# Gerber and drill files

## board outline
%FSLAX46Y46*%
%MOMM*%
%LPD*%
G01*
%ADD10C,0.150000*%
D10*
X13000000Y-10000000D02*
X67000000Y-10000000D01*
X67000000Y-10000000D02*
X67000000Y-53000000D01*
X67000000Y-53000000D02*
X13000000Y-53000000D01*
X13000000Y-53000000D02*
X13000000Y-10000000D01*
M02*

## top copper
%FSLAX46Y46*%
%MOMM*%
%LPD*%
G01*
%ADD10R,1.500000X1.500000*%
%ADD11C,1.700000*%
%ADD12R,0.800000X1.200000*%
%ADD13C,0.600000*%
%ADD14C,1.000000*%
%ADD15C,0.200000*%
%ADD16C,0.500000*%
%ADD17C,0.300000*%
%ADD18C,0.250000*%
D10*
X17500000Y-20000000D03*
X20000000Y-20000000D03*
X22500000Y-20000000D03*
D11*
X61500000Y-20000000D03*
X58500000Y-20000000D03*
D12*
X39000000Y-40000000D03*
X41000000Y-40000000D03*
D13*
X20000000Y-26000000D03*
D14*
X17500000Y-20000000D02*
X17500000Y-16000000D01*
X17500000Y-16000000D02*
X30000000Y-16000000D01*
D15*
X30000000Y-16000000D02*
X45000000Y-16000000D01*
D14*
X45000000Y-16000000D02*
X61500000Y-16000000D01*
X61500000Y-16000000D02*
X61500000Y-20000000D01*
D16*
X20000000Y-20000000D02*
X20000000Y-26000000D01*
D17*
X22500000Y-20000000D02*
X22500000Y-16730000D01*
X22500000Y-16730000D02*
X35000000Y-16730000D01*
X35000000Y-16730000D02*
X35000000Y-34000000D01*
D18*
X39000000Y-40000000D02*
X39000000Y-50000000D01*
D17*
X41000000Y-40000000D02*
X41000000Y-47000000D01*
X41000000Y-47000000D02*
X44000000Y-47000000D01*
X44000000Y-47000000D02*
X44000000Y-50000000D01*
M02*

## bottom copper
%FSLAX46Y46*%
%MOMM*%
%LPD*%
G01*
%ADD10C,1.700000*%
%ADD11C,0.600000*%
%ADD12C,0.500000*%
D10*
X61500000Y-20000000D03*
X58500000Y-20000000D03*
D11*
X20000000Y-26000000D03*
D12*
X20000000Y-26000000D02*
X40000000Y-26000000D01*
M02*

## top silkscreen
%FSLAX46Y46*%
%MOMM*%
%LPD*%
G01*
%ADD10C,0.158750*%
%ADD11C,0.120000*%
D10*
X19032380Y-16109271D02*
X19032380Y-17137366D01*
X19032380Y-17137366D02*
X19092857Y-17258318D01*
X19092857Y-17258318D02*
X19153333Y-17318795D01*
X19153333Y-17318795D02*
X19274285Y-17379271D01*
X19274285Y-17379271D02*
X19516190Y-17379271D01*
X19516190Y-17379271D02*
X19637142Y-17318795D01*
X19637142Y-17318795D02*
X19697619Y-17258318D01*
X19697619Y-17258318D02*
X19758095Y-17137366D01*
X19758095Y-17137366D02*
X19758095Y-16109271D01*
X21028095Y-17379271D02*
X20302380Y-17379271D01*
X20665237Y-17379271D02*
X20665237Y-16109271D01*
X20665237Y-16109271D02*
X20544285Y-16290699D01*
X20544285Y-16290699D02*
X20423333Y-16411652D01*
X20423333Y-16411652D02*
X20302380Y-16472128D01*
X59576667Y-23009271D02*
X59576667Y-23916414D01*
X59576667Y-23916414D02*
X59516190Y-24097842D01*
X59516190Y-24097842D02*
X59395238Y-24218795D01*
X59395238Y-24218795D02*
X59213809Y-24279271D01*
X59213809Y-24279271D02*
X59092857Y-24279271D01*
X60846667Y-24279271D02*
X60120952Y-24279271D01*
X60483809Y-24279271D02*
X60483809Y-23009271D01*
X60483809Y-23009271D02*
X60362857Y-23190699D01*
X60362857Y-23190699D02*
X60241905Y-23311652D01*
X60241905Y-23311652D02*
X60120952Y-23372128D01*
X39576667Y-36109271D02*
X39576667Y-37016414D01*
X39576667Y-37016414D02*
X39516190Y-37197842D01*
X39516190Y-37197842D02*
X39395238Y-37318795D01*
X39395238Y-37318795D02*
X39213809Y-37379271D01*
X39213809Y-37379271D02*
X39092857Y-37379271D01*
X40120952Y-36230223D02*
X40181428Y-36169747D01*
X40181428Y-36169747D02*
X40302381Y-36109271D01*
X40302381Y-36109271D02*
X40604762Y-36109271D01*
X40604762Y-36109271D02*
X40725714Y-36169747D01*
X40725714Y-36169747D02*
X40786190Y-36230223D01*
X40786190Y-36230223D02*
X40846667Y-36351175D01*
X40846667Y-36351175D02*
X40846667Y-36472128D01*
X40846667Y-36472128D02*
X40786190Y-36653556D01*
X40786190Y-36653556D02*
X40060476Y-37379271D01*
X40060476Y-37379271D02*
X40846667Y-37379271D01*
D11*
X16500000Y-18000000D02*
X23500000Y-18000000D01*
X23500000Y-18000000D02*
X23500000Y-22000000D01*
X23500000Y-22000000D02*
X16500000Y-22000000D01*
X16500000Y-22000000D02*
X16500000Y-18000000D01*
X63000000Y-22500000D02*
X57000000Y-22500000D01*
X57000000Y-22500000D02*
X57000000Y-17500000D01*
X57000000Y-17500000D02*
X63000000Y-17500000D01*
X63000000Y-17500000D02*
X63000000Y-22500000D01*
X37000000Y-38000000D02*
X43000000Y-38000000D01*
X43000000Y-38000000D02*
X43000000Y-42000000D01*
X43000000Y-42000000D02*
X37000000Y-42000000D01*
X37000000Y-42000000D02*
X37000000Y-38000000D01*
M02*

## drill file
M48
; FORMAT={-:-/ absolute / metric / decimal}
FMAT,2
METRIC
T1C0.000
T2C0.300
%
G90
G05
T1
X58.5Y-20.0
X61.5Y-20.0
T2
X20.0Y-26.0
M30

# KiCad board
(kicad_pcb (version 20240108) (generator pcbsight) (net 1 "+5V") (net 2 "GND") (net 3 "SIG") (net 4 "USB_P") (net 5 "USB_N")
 (gr_line (start 13 10) (end 67 10) (layer "Edge.Cuts") (width 0.15))
 (gr_line (start 67 10) (end 67 53) (layer "Edge.Cuts") (width 0.15))
 (gr_line (start 67 53) (end 13 53) (layer "Edge.Cuts") (width 0.15))
 (gr_line (start 13 53) (end 13 10) (layer "Edge.Cuts") (width 0.15))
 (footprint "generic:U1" (at 20 20 0) (layer "F.Cu") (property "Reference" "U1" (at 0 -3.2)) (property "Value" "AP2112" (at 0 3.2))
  (fp_line (start -3.5 -2.0) (end 3.5 -2.0) (layer "F.SilkS") (width 0.12))
  (fp_line (start 3.5 -2.0) (end 3.5 2.0) (layer "F.SilkS") (width 0.12))
  (fp_line (start 3.5 2.0) (end -3.5 2.0) (layer "F.SilkS") (width 0.12))
  (fp_line (start -3.5 2.0) (end -3.5 -2.0) (layer "F.SilkS") (width 0.12))
  (pad "1" smd rect (at -2.5 0) (size 1.5 1.5) (layers "F.Cu" "F.Mask") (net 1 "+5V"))
  (pad "2" smd rect (at 0 0) (size 1.5 1.5) (layers "F.Cu" "F.Mask") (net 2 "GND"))
  (pad "3" smd rect (at 2.5 0) (size 1.5 1.5) (layers "F.Cu" "F.Mask") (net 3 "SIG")))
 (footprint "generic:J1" (at 60 20 180) (layer "F.Cu") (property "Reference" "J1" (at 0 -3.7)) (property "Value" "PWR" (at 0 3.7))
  (fp_line (start -3.0 -2.5) (end 3.0 -2.5) (layer "F.SilkS") (width 0.12))
  (fp_line (start 3.0 -2.5) (end 3.0 2.5) (layer "F.SilkS") (width 0.12))
  (fp_line (start 3.0 2.5) (end -3.0 2.5) (layer "F.SilkS") (width 0.12))
  (fp_line (start -3.0 2.5) (end -3.0 -2.5) (layer "F.SilkS") (width 0.12))
  (pad "1" thru_hole circle (at -1.5 0) (size 1.7 1.7) (layers "*.Cu" "*.Mask") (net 1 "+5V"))
  (pad "2" thru_hole circle (at 1.5 0) (size 1.7 1.7) (layers "*.Cu" "*.Mask") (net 2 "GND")))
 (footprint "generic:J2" (at 40 40 0) (layer "F.Cu") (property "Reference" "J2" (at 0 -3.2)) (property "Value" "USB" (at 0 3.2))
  (fp_line (start -3.0 -2.0) (end 3.0 -2.0) (layer "F.SilkS") (width 0.12))
  (fp_line (start 3.0 -2.0) (end 3.0 2.0) (layer "F.SilkS") (width 0.12))
  (fp_line (start 3.0 2.0) (end -3.0 2.0) (layer "F.SilkS") (width 0.12))
  (fp_line (start -3.0 2.0) (end -3.0 -2.0) (layer "F.SilkS") (width 0.12))
  (pad "1" smd rect (at -1.0 0) (size 0.8 1.2) (layers "F.Cu" "F.Mask") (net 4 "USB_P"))
  (pad "2" smd rect (at 1.0 0) (size 0.8 1.2) (layers "F.Cu" "F.Mask") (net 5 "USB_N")))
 (segment (start 17.5 20) (end 17.5 16) (width 1.0) (layer "F.Cu") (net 1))
 (segment (start 17.5 16) (end 30 16) (width 1.0) (layer "F.Cu") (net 1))
 (segment (start 30 16) (end 45 16) (width 0.2) (layer "F.Cu") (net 1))
 (segment (start 45 16) (end 61.5 16) (width 1.0) (layer "F.Cu") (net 1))
 (segment (start 61.5 16) (end 61.5 20) (width 1.0) (layer "F.Cu") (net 1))
 (segment (start 20 20) (end 20 26) (width 0.5) (layer "F.Cu") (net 2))
 (via (at 20 26) (size 0.6) (drill 0.3) (layers "F.Cu" "B.Cu") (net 2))
 (segment (start 20 26) (end 40 26) (width 0.5) (layer "B.Cu") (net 2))
 (segment (start 22.5 20) (end 22.5 16.73) (width 0.3) (layer "F.Cu") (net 3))
 (segment (start 22.5 16.73) (end 35 16.73) (width 0.3) (layer "F.Cu") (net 3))
 (segment (start 35 16.73) (end 35 34) (width 0.3) (layer "F.Cu") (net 3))
 (segment (start 39 40) (end 39 50) (width 0.25) (layer "F.Cu") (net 4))
 (segment (start 41 40) (end 41 47) (width 0.3) (layer "F.Cu") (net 5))
 (segment (start 41 47) (end 44 47) (width 0.3) (layer "F.Cu") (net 5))
 (segment (start 44 47) (end 44 50) (width 0.3) (layer "F.Cu") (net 5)))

